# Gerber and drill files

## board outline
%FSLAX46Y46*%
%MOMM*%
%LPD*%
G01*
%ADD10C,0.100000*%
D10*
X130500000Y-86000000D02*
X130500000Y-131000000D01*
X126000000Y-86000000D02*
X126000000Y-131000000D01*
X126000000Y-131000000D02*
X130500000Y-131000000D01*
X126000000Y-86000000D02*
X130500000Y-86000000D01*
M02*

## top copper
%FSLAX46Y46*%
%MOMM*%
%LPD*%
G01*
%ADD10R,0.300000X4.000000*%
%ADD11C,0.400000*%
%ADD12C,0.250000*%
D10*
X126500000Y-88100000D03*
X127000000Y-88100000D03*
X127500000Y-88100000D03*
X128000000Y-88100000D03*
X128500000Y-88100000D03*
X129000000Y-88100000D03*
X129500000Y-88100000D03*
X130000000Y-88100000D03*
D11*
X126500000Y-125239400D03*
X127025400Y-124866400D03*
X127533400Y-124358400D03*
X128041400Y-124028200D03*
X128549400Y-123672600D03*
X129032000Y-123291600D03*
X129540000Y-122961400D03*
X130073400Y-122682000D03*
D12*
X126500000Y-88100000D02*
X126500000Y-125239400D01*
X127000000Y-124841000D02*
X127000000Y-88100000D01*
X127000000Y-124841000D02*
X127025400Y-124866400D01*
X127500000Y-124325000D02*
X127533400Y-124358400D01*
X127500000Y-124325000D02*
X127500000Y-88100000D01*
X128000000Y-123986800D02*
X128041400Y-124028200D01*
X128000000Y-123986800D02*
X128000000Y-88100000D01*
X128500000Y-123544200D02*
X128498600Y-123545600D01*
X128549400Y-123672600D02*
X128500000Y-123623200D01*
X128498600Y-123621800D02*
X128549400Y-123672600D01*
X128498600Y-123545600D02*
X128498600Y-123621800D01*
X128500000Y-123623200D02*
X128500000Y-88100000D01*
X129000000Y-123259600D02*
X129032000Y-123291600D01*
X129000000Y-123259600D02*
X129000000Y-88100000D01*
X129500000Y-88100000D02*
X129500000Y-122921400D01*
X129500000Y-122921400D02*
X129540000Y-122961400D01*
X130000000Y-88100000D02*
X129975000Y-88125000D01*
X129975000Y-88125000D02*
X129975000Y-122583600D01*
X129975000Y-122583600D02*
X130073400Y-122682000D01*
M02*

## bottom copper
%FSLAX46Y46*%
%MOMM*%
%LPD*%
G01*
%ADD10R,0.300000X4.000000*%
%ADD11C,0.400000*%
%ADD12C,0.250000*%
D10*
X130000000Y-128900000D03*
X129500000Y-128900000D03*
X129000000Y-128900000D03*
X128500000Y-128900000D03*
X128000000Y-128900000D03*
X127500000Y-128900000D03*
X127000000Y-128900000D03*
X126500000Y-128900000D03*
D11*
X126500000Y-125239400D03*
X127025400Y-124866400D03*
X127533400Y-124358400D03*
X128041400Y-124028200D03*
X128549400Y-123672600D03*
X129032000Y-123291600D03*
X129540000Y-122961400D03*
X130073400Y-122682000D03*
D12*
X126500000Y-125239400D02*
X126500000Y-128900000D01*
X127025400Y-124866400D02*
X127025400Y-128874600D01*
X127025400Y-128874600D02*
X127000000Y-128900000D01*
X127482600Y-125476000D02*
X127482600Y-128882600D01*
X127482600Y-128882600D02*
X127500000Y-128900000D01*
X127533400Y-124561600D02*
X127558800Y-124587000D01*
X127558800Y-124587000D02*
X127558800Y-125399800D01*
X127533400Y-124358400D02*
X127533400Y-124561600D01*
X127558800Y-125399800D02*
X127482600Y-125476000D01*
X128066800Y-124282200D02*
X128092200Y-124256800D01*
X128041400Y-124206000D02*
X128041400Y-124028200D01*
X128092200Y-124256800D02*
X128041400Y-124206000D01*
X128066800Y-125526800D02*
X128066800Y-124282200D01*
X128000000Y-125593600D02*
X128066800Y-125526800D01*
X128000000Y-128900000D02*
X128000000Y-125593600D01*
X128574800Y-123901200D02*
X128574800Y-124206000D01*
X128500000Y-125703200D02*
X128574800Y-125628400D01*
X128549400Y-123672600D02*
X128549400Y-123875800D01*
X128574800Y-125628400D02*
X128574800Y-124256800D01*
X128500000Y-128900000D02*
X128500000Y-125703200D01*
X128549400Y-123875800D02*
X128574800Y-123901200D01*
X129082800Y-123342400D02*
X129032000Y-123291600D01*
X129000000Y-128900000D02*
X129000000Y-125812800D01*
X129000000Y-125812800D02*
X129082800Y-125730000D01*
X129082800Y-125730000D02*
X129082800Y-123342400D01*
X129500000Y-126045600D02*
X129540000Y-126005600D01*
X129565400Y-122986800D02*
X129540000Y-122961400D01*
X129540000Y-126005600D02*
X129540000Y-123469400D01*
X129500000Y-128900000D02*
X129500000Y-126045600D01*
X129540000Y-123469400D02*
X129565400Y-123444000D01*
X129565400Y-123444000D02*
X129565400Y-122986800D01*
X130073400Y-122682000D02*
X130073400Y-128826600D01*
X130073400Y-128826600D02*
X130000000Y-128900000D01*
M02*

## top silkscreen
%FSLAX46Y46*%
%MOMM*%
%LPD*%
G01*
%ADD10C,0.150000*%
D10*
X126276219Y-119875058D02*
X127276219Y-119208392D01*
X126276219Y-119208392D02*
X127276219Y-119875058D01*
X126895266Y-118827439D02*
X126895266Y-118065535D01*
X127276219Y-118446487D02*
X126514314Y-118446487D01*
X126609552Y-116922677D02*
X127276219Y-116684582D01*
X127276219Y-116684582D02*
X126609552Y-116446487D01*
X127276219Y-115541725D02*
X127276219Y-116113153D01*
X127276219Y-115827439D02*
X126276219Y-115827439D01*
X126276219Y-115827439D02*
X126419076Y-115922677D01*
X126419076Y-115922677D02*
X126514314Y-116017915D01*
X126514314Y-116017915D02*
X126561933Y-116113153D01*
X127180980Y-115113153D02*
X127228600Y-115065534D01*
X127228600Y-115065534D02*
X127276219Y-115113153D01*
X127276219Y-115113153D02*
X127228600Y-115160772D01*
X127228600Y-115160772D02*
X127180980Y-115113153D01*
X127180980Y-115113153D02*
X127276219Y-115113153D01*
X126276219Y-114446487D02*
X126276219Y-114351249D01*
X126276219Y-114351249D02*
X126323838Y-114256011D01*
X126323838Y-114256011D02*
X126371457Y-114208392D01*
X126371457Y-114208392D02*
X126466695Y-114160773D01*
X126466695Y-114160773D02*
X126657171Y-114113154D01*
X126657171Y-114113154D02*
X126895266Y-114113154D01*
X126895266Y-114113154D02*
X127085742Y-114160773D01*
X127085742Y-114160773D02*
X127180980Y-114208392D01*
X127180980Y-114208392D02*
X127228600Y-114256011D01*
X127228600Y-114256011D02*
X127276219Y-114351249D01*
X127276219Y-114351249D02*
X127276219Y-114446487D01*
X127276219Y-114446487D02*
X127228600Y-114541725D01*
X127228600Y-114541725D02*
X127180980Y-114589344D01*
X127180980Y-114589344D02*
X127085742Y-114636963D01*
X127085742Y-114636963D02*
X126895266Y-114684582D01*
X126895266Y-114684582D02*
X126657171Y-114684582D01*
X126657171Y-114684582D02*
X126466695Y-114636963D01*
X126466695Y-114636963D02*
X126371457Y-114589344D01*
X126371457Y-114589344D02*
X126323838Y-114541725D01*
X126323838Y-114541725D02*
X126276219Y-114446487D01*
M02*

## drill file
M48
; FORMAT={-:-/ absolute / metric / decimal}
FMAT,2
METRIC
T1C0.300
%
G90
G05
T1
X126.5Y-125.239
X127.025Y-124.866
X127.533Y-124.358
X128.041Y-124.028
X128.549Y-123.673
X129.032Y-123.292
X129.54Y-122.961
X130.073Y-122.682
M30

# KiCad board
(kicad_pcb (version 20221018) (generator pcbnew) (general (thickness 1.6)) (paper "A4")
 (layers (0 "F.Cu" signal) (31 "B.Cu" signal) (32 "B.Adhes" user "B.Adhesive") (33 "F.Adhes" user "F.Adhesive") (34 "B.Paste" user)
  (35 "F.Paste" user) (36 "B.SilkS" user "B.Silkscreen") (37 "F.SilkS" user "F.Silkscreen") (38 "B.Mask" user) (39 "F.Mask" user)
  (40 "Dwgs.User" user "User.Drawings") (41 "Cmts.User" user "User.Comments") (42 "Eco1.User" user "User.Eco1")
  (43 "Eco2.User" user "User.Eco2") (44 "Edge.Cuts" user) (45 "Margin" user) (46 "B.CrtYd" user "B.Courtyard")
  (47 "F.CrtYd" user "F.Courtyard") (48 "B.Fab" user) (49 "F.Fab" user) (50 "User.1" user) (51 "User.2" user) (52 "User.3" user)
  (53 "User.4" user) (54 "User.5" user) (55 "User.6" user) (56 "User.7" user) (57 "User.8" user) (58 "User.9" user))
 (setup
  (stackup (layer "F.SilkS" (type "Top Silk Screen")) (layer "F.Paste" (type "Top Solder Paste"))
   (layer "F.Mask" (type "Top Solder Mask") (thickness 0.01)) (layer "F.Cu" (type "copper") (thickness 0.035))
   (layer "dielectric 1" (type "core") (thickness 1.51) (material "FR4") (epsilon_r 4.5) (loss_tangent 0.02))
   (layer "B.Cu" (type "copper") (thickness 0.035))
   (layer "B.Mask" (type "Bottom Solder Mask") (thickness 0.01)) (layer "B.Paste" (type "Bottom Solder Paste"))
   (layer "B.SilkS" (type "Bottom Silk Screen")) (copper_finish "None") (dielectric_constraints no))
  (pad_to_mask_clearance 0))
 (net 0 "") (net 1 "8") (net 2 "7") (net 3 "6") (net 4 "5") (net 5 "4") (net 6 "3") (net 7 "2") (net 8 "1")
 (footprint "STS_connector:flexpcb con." (layer "F.Cu") (at 126 90.1)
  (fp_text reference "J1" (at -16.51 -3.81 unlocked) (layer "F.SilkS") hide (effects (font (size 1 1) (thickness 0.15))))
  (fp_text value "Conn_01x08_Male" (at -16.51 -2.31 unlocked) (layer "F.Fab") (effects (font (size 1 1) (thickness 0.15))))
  (pad "1" smd rect (at 0.5 -2) (size 0.3 4) (layers "F.Cu" "F.Paste" "F.Mask") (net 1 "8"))
  (pad "2" smd rect (at 1 -2) (size 0.3 4) (layers "F.Cu" "F.Paste" "F.Mask") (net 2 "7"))
  (pad "3" smd rect (at 1.5 -2) (size 0.3 4) (layers "F.Cu" "F.Paste" "F.Mask") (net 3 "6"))
  (pad "4" smd rect (at 2 -2) (size 0.3 4) (layers "F.Cu" "F.Paste" "F.Mask") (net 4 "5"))
  (pad "5" smd rect (at 2.5 -2) (size 0.3 4) (layers "F.Cu" "F.Paste" "F.Mask") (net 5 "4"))
  (pad "6" smd rect (at 3 -2) (size 0.3 4) (layers "F.Cu" "F.Paste" "F.Mask") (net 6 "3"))
  (pad "7" smd rect (at 3.5 -2) (size 0.3 4) (layers "F.Cu" "F.Paste" "F.Mask") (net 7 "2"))
  (pad "8" smd rect (at 4 -2) (size 0.3 4) (layers "F.Cu" "F.Paste" "F.Mask") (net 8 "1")))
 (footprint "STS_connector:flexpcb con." (layer "B.Cu") (at 130.5 130.9 180)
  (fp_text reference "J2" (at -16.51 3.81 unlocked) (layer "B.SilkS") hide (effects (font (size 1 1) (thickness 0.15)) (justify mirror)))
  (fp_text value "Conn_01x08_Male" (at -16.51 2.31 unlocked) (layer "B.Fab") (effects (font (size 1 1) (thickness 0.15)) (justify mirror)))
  (pad "1" smd rect (at 0.5 2 180) (size 0.3 4) (layers "B.Cu" "B.Paste" "B.Mask") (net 8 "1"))
  (pad "2" smd rect (at 1 2 180) (size 0.3 4) (layers "B.Cu" "B.Paste" "B.Mask") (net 7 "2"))
  (pad "3" smd rect (at 1.5 2 180) (size 0.3 4) (layers "B.Cu" "B.Paste" "B.Mask") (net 6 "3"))
  (pad "4" smd rect (at 2 2 180) (size 0.3 4) (layers "B.Cu" "B.Paste" "B.Mask") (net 5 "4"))
  (pad "5" smd rect (at 2.5 2 180) (size 0.3 4) (layers "B.Cu" "B.Paste" "B.Mask") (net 4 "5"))
  (pad "6" smd rect (at 3 2 180) (size 0.3 4) (layers "B.Cu" "B.Paste" "B.Mask") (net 3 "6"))
  (pad "7" smd rect (at 3.5 2 180) (size 0.3 4) (layers "B.Cu" "B.Paste" "B.Mask") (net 2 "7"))
  (pad "8" smd rect (at 4 2 180) (size 0.3 4) (layers "B.Cu" "B.Paste" "B.Mask") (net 1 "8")))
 (gr_line (start 130.5 86) (end 130.5 131) (stroke (width 0.1) (type solid)) (layer "Edge.Cuts"))
 (gr_line (start 126 86) (end 126 131) (stroke (width 0.1) (type solid)) (layer "Edge.Cuts"))
 (gr_line (start 126 131) (end 130.5 131) (stroke (width 0.1) (type solid)) (layer "Edge.Cuts"))
 (gr_line (start 126 86) (end 130.5 86) (stroke (width 0.1) (type solid)) (layer "Edge.Cuts"))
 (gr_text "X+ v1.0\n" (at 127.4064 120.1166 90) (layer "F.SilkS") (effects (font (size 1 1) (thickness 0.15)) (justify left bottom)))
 (segment (start 126.5 88.1) (end 126.5 125.2394) (width 0.25) (layer "F.Cu") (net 1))
 (via (at 126.5 125.2394) (size 0.4) (drill 0.3) (layers "F.Cu" "B.Cu") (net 1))
 (segment (start 126.5 125.2394) (end 126.5 128.9) (width 0.25) (layer "B.Cu") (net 1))
 (segment (start 127 124.841) (end 127 88.1) (width 0.25) (layer "F.Cu") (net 2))
 (segment (start 127 124.841) (end 127.0254 124.8664) (width 0.25) (layer "F.Cu") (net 2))
 (via (at 127.0254 124.8664) (size 0.4) (drill 0.3) (layers "F.Cu" "B.Cu") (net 2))
 (segment (start 127.0254 124.8664) (end 127.0254 128.8746) (width 0.25) (layer "B.Cu") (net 2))
 (segment (start 127.0254 128.8746) (end 127 128.9) (width 0.25) (layer "B.Cu") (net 2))
 (segment (start 127.5 124.325) (end 127.5334 124.3584) (width 0.25) (layer "F.Cu") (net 3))
 (segment (start 127.5 124.325) (end 127.5 88.1) (width 0.25) (layer "F.Cu") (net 3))
 (via (at 127.5334 124.3584) (size 0.4) (drill 0.3) (layers "F.Cu" "B.Cu") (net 3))
 (segment (start 127.4826 125.476) (end 127.4826 128.8826) (width 0.25) (layer "B.Cu") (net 3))
 (segment (start 127.4826 128.8826) (end 127.5 128.9) (width 0.25) (layer "B.Cu") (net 3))
 (segment (start 127.5334 124.5616) (end 127.5588 124.587) (width 0.25) (layer "B.Cu") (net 3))
 (segment (start 127.5588 124.587) (end 127.5588 125.3998) (width 0.25) (layer "B.Cu") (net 3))
 (segment (start 127.5334 124.3584) (end 127.5334 124.5616) (width 0.25) (layer "B.Cu") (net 3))
 (segment (start 127.5588 125.3998) (end 127.4826 125.476) (width 0.25) (layer "B.Cu") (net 3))
 (segment (start 128 123.9868) (end 128.0414 124.0282) (width 0.25) (layer "F.Cu") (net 4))
 (segment (start 128 123.9868) (end 128 88.1) (width 0.25) (layer "F.Cu") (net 4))
 (via (at 128.0414 124.0282) (size 0.4) (drill 0.3) (layers "F.Cu" "B.Cu") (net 4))
 (segment (start 128.0668 124.2822) (end 128.0922 124.2568) (width 0.25) (layer "B.Cu") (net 4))
 (segment (start 128.0414 124.206) (end 128.0414 124.0282) (width 0.25) (layer "B.Cu") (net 4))
 (segment (start 128.0922 124.2568) (end 128.0414 124.206) (width 0.25) (layer "B.Cu") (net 4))
 (segment (start 128.0668 125.5268) (end 128.0668 124.2822) (width 0.25) (layer "B.Cu") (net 4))
 (segment (start 128 125.5936) (end 128.0668 125.5268) (width 0.25) (layer "B.Cu") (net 4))
 (segment (start 128 128.9) (end 128 125.5936) (width 0.25) (layer "B.Cu") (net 4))
 (segment (start 128.5 123.5442) (end 128.4986 123.5456) (width 0.25) (layer "F.Cu") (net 5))
 (segment (start 128.5494 123.6726) (end 128.5 123.6232) (width 0.25) (layer "F.Cu") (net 5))
 (segment (start 128.4986 123.6218) (end 128.5494 123.6726) (width 0.25) (layer "F.Cu") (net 5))
 (segment (start 128.4986 123.5456) (end 128.4986 123.6218) (width 0.25) (layer "F.Cu") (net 5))
 (segment (start 128.5 123.6232) (end 128.5 88.1) (width 0.25) (layer "F.Cu") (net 5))
 (via (at 128.5494 123.6726) (size 0.4) (drill 0.3) (layers "F.Cu" "B.Cu") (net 5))
 (segment (start 128.5748 123.9012) (end 128.5748 124.206) (width 0.25) (layer "B.Cu") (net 5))
 (segment (start 128.5 125.7032) (end 128.5748 125.6284) (width 0.25) (layer "B.Cu") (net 5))
 (segment (start 128.5494 123.6726) (end 128.5494 123.8758) (width 0.25) (layer "B.Cu") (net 5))
 (segment (start 128.5748 125.6284) (end 128.5748 124.2568) (width 0.25) (layer "B.Cu") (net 5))
 (segment (start 128.5 128.9) (end 128.5 125.7032) (width 0.25) (layer "B.Cu") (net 5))
 (segment (start 128.5494 123.8758) (end 128.5748 123.9012) (width 0.25) (layer "B.Cu") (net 5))
 (segment (start 129 123.2596) (end 129.032 123.2916) (width 0.25) (layer "F.Cu") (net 6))
 (segment (start 129 123.2596) (end 129 88.1) (width 0.25) (layer "F.Cu") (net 6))
 (via (at 129.032 123.2916) (size 0.4) (drill 0.3) (layers "F.Cu" "B.Cu") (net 6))
 (segment (start 129.0828 123.3424) (end 129.032 123.2916) (width 0.25) (layer "B.Cu") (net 6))
 (segment (start 129 128.9) (end 129 125.8128) (width 0.25) (layer "B.Cu") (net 6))
 (segment (start 129 125.8128) (end 129.0828 125.73) (width 0.25) (layer "B.Cu") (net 6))
 (segment (start 129.0828 125.73) (end 129.0828 123.3424) (width 0.25) (layer "B.Cu") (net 6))
 (segment (start 129.5 88.1) (end 129.5 122.9214) (width 0.25) (layer "F.Cu") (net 7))
 (segment (start 129.5 122.9214) (end 129.54 122.9614) (width 0.25) (layer "F.Cu") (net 7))
 (via (at 129.54 122.9614) (size 0.4) (drill 0.3) (layers "F.Cu" "B.Cu") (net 7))
 (segment (start 129.5 126.0456) (end 129.54 126.0056) (width 0.25) (layer "B.Cu") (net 7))
 (segment (start 129.5654 122.9868) (end 129.54 122.9614) (width 0.25) (layer "B.Cu") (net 7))
 (segment (start 129.54 126.0056) (end 129.54 123.4694) (width 0.25) (layer "B.Cu") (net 7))
 (segment (start 129.5 128.9) (end 129.5 126.0456) (width 0.25) (layer "B.Cu") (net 7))
 (segment (start 129.54 123.4694) (end 129.5654 123.444) (width 0.25) (layer "B.Cu") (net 7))
 (segment (start 129.5654 123.444) (end 129.5654 122.9868) (width 0.25) (layer "B.Cu") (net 7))
 (segment (start 130 88.1) (end 129.975 88.125) (width 0.25) (layer "F.Cu") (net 8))
 (segment (start 129.975 88.125) (end 129.975 122.5836) (width 0.25) (layer "F.Cu") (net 8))
 (segment (start 129.975 122.5836) (end 130.0734 122.682) (width 0.25) (layer "F.Cu") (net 8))
 (via (at 130.0734 122.682) (size 0.4) (drill 0.3) (layers "F.Cu" "B.Cu") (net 8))
 (segment (start 130.0734 122.682) (end 130.0734 128.8266) (width 0.25) (layer "B.Cu") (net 8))
 (segment (start 130.0734 128.8266) (end 130 128.9) (width 0.25) (layer "B.Cu") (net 8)))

